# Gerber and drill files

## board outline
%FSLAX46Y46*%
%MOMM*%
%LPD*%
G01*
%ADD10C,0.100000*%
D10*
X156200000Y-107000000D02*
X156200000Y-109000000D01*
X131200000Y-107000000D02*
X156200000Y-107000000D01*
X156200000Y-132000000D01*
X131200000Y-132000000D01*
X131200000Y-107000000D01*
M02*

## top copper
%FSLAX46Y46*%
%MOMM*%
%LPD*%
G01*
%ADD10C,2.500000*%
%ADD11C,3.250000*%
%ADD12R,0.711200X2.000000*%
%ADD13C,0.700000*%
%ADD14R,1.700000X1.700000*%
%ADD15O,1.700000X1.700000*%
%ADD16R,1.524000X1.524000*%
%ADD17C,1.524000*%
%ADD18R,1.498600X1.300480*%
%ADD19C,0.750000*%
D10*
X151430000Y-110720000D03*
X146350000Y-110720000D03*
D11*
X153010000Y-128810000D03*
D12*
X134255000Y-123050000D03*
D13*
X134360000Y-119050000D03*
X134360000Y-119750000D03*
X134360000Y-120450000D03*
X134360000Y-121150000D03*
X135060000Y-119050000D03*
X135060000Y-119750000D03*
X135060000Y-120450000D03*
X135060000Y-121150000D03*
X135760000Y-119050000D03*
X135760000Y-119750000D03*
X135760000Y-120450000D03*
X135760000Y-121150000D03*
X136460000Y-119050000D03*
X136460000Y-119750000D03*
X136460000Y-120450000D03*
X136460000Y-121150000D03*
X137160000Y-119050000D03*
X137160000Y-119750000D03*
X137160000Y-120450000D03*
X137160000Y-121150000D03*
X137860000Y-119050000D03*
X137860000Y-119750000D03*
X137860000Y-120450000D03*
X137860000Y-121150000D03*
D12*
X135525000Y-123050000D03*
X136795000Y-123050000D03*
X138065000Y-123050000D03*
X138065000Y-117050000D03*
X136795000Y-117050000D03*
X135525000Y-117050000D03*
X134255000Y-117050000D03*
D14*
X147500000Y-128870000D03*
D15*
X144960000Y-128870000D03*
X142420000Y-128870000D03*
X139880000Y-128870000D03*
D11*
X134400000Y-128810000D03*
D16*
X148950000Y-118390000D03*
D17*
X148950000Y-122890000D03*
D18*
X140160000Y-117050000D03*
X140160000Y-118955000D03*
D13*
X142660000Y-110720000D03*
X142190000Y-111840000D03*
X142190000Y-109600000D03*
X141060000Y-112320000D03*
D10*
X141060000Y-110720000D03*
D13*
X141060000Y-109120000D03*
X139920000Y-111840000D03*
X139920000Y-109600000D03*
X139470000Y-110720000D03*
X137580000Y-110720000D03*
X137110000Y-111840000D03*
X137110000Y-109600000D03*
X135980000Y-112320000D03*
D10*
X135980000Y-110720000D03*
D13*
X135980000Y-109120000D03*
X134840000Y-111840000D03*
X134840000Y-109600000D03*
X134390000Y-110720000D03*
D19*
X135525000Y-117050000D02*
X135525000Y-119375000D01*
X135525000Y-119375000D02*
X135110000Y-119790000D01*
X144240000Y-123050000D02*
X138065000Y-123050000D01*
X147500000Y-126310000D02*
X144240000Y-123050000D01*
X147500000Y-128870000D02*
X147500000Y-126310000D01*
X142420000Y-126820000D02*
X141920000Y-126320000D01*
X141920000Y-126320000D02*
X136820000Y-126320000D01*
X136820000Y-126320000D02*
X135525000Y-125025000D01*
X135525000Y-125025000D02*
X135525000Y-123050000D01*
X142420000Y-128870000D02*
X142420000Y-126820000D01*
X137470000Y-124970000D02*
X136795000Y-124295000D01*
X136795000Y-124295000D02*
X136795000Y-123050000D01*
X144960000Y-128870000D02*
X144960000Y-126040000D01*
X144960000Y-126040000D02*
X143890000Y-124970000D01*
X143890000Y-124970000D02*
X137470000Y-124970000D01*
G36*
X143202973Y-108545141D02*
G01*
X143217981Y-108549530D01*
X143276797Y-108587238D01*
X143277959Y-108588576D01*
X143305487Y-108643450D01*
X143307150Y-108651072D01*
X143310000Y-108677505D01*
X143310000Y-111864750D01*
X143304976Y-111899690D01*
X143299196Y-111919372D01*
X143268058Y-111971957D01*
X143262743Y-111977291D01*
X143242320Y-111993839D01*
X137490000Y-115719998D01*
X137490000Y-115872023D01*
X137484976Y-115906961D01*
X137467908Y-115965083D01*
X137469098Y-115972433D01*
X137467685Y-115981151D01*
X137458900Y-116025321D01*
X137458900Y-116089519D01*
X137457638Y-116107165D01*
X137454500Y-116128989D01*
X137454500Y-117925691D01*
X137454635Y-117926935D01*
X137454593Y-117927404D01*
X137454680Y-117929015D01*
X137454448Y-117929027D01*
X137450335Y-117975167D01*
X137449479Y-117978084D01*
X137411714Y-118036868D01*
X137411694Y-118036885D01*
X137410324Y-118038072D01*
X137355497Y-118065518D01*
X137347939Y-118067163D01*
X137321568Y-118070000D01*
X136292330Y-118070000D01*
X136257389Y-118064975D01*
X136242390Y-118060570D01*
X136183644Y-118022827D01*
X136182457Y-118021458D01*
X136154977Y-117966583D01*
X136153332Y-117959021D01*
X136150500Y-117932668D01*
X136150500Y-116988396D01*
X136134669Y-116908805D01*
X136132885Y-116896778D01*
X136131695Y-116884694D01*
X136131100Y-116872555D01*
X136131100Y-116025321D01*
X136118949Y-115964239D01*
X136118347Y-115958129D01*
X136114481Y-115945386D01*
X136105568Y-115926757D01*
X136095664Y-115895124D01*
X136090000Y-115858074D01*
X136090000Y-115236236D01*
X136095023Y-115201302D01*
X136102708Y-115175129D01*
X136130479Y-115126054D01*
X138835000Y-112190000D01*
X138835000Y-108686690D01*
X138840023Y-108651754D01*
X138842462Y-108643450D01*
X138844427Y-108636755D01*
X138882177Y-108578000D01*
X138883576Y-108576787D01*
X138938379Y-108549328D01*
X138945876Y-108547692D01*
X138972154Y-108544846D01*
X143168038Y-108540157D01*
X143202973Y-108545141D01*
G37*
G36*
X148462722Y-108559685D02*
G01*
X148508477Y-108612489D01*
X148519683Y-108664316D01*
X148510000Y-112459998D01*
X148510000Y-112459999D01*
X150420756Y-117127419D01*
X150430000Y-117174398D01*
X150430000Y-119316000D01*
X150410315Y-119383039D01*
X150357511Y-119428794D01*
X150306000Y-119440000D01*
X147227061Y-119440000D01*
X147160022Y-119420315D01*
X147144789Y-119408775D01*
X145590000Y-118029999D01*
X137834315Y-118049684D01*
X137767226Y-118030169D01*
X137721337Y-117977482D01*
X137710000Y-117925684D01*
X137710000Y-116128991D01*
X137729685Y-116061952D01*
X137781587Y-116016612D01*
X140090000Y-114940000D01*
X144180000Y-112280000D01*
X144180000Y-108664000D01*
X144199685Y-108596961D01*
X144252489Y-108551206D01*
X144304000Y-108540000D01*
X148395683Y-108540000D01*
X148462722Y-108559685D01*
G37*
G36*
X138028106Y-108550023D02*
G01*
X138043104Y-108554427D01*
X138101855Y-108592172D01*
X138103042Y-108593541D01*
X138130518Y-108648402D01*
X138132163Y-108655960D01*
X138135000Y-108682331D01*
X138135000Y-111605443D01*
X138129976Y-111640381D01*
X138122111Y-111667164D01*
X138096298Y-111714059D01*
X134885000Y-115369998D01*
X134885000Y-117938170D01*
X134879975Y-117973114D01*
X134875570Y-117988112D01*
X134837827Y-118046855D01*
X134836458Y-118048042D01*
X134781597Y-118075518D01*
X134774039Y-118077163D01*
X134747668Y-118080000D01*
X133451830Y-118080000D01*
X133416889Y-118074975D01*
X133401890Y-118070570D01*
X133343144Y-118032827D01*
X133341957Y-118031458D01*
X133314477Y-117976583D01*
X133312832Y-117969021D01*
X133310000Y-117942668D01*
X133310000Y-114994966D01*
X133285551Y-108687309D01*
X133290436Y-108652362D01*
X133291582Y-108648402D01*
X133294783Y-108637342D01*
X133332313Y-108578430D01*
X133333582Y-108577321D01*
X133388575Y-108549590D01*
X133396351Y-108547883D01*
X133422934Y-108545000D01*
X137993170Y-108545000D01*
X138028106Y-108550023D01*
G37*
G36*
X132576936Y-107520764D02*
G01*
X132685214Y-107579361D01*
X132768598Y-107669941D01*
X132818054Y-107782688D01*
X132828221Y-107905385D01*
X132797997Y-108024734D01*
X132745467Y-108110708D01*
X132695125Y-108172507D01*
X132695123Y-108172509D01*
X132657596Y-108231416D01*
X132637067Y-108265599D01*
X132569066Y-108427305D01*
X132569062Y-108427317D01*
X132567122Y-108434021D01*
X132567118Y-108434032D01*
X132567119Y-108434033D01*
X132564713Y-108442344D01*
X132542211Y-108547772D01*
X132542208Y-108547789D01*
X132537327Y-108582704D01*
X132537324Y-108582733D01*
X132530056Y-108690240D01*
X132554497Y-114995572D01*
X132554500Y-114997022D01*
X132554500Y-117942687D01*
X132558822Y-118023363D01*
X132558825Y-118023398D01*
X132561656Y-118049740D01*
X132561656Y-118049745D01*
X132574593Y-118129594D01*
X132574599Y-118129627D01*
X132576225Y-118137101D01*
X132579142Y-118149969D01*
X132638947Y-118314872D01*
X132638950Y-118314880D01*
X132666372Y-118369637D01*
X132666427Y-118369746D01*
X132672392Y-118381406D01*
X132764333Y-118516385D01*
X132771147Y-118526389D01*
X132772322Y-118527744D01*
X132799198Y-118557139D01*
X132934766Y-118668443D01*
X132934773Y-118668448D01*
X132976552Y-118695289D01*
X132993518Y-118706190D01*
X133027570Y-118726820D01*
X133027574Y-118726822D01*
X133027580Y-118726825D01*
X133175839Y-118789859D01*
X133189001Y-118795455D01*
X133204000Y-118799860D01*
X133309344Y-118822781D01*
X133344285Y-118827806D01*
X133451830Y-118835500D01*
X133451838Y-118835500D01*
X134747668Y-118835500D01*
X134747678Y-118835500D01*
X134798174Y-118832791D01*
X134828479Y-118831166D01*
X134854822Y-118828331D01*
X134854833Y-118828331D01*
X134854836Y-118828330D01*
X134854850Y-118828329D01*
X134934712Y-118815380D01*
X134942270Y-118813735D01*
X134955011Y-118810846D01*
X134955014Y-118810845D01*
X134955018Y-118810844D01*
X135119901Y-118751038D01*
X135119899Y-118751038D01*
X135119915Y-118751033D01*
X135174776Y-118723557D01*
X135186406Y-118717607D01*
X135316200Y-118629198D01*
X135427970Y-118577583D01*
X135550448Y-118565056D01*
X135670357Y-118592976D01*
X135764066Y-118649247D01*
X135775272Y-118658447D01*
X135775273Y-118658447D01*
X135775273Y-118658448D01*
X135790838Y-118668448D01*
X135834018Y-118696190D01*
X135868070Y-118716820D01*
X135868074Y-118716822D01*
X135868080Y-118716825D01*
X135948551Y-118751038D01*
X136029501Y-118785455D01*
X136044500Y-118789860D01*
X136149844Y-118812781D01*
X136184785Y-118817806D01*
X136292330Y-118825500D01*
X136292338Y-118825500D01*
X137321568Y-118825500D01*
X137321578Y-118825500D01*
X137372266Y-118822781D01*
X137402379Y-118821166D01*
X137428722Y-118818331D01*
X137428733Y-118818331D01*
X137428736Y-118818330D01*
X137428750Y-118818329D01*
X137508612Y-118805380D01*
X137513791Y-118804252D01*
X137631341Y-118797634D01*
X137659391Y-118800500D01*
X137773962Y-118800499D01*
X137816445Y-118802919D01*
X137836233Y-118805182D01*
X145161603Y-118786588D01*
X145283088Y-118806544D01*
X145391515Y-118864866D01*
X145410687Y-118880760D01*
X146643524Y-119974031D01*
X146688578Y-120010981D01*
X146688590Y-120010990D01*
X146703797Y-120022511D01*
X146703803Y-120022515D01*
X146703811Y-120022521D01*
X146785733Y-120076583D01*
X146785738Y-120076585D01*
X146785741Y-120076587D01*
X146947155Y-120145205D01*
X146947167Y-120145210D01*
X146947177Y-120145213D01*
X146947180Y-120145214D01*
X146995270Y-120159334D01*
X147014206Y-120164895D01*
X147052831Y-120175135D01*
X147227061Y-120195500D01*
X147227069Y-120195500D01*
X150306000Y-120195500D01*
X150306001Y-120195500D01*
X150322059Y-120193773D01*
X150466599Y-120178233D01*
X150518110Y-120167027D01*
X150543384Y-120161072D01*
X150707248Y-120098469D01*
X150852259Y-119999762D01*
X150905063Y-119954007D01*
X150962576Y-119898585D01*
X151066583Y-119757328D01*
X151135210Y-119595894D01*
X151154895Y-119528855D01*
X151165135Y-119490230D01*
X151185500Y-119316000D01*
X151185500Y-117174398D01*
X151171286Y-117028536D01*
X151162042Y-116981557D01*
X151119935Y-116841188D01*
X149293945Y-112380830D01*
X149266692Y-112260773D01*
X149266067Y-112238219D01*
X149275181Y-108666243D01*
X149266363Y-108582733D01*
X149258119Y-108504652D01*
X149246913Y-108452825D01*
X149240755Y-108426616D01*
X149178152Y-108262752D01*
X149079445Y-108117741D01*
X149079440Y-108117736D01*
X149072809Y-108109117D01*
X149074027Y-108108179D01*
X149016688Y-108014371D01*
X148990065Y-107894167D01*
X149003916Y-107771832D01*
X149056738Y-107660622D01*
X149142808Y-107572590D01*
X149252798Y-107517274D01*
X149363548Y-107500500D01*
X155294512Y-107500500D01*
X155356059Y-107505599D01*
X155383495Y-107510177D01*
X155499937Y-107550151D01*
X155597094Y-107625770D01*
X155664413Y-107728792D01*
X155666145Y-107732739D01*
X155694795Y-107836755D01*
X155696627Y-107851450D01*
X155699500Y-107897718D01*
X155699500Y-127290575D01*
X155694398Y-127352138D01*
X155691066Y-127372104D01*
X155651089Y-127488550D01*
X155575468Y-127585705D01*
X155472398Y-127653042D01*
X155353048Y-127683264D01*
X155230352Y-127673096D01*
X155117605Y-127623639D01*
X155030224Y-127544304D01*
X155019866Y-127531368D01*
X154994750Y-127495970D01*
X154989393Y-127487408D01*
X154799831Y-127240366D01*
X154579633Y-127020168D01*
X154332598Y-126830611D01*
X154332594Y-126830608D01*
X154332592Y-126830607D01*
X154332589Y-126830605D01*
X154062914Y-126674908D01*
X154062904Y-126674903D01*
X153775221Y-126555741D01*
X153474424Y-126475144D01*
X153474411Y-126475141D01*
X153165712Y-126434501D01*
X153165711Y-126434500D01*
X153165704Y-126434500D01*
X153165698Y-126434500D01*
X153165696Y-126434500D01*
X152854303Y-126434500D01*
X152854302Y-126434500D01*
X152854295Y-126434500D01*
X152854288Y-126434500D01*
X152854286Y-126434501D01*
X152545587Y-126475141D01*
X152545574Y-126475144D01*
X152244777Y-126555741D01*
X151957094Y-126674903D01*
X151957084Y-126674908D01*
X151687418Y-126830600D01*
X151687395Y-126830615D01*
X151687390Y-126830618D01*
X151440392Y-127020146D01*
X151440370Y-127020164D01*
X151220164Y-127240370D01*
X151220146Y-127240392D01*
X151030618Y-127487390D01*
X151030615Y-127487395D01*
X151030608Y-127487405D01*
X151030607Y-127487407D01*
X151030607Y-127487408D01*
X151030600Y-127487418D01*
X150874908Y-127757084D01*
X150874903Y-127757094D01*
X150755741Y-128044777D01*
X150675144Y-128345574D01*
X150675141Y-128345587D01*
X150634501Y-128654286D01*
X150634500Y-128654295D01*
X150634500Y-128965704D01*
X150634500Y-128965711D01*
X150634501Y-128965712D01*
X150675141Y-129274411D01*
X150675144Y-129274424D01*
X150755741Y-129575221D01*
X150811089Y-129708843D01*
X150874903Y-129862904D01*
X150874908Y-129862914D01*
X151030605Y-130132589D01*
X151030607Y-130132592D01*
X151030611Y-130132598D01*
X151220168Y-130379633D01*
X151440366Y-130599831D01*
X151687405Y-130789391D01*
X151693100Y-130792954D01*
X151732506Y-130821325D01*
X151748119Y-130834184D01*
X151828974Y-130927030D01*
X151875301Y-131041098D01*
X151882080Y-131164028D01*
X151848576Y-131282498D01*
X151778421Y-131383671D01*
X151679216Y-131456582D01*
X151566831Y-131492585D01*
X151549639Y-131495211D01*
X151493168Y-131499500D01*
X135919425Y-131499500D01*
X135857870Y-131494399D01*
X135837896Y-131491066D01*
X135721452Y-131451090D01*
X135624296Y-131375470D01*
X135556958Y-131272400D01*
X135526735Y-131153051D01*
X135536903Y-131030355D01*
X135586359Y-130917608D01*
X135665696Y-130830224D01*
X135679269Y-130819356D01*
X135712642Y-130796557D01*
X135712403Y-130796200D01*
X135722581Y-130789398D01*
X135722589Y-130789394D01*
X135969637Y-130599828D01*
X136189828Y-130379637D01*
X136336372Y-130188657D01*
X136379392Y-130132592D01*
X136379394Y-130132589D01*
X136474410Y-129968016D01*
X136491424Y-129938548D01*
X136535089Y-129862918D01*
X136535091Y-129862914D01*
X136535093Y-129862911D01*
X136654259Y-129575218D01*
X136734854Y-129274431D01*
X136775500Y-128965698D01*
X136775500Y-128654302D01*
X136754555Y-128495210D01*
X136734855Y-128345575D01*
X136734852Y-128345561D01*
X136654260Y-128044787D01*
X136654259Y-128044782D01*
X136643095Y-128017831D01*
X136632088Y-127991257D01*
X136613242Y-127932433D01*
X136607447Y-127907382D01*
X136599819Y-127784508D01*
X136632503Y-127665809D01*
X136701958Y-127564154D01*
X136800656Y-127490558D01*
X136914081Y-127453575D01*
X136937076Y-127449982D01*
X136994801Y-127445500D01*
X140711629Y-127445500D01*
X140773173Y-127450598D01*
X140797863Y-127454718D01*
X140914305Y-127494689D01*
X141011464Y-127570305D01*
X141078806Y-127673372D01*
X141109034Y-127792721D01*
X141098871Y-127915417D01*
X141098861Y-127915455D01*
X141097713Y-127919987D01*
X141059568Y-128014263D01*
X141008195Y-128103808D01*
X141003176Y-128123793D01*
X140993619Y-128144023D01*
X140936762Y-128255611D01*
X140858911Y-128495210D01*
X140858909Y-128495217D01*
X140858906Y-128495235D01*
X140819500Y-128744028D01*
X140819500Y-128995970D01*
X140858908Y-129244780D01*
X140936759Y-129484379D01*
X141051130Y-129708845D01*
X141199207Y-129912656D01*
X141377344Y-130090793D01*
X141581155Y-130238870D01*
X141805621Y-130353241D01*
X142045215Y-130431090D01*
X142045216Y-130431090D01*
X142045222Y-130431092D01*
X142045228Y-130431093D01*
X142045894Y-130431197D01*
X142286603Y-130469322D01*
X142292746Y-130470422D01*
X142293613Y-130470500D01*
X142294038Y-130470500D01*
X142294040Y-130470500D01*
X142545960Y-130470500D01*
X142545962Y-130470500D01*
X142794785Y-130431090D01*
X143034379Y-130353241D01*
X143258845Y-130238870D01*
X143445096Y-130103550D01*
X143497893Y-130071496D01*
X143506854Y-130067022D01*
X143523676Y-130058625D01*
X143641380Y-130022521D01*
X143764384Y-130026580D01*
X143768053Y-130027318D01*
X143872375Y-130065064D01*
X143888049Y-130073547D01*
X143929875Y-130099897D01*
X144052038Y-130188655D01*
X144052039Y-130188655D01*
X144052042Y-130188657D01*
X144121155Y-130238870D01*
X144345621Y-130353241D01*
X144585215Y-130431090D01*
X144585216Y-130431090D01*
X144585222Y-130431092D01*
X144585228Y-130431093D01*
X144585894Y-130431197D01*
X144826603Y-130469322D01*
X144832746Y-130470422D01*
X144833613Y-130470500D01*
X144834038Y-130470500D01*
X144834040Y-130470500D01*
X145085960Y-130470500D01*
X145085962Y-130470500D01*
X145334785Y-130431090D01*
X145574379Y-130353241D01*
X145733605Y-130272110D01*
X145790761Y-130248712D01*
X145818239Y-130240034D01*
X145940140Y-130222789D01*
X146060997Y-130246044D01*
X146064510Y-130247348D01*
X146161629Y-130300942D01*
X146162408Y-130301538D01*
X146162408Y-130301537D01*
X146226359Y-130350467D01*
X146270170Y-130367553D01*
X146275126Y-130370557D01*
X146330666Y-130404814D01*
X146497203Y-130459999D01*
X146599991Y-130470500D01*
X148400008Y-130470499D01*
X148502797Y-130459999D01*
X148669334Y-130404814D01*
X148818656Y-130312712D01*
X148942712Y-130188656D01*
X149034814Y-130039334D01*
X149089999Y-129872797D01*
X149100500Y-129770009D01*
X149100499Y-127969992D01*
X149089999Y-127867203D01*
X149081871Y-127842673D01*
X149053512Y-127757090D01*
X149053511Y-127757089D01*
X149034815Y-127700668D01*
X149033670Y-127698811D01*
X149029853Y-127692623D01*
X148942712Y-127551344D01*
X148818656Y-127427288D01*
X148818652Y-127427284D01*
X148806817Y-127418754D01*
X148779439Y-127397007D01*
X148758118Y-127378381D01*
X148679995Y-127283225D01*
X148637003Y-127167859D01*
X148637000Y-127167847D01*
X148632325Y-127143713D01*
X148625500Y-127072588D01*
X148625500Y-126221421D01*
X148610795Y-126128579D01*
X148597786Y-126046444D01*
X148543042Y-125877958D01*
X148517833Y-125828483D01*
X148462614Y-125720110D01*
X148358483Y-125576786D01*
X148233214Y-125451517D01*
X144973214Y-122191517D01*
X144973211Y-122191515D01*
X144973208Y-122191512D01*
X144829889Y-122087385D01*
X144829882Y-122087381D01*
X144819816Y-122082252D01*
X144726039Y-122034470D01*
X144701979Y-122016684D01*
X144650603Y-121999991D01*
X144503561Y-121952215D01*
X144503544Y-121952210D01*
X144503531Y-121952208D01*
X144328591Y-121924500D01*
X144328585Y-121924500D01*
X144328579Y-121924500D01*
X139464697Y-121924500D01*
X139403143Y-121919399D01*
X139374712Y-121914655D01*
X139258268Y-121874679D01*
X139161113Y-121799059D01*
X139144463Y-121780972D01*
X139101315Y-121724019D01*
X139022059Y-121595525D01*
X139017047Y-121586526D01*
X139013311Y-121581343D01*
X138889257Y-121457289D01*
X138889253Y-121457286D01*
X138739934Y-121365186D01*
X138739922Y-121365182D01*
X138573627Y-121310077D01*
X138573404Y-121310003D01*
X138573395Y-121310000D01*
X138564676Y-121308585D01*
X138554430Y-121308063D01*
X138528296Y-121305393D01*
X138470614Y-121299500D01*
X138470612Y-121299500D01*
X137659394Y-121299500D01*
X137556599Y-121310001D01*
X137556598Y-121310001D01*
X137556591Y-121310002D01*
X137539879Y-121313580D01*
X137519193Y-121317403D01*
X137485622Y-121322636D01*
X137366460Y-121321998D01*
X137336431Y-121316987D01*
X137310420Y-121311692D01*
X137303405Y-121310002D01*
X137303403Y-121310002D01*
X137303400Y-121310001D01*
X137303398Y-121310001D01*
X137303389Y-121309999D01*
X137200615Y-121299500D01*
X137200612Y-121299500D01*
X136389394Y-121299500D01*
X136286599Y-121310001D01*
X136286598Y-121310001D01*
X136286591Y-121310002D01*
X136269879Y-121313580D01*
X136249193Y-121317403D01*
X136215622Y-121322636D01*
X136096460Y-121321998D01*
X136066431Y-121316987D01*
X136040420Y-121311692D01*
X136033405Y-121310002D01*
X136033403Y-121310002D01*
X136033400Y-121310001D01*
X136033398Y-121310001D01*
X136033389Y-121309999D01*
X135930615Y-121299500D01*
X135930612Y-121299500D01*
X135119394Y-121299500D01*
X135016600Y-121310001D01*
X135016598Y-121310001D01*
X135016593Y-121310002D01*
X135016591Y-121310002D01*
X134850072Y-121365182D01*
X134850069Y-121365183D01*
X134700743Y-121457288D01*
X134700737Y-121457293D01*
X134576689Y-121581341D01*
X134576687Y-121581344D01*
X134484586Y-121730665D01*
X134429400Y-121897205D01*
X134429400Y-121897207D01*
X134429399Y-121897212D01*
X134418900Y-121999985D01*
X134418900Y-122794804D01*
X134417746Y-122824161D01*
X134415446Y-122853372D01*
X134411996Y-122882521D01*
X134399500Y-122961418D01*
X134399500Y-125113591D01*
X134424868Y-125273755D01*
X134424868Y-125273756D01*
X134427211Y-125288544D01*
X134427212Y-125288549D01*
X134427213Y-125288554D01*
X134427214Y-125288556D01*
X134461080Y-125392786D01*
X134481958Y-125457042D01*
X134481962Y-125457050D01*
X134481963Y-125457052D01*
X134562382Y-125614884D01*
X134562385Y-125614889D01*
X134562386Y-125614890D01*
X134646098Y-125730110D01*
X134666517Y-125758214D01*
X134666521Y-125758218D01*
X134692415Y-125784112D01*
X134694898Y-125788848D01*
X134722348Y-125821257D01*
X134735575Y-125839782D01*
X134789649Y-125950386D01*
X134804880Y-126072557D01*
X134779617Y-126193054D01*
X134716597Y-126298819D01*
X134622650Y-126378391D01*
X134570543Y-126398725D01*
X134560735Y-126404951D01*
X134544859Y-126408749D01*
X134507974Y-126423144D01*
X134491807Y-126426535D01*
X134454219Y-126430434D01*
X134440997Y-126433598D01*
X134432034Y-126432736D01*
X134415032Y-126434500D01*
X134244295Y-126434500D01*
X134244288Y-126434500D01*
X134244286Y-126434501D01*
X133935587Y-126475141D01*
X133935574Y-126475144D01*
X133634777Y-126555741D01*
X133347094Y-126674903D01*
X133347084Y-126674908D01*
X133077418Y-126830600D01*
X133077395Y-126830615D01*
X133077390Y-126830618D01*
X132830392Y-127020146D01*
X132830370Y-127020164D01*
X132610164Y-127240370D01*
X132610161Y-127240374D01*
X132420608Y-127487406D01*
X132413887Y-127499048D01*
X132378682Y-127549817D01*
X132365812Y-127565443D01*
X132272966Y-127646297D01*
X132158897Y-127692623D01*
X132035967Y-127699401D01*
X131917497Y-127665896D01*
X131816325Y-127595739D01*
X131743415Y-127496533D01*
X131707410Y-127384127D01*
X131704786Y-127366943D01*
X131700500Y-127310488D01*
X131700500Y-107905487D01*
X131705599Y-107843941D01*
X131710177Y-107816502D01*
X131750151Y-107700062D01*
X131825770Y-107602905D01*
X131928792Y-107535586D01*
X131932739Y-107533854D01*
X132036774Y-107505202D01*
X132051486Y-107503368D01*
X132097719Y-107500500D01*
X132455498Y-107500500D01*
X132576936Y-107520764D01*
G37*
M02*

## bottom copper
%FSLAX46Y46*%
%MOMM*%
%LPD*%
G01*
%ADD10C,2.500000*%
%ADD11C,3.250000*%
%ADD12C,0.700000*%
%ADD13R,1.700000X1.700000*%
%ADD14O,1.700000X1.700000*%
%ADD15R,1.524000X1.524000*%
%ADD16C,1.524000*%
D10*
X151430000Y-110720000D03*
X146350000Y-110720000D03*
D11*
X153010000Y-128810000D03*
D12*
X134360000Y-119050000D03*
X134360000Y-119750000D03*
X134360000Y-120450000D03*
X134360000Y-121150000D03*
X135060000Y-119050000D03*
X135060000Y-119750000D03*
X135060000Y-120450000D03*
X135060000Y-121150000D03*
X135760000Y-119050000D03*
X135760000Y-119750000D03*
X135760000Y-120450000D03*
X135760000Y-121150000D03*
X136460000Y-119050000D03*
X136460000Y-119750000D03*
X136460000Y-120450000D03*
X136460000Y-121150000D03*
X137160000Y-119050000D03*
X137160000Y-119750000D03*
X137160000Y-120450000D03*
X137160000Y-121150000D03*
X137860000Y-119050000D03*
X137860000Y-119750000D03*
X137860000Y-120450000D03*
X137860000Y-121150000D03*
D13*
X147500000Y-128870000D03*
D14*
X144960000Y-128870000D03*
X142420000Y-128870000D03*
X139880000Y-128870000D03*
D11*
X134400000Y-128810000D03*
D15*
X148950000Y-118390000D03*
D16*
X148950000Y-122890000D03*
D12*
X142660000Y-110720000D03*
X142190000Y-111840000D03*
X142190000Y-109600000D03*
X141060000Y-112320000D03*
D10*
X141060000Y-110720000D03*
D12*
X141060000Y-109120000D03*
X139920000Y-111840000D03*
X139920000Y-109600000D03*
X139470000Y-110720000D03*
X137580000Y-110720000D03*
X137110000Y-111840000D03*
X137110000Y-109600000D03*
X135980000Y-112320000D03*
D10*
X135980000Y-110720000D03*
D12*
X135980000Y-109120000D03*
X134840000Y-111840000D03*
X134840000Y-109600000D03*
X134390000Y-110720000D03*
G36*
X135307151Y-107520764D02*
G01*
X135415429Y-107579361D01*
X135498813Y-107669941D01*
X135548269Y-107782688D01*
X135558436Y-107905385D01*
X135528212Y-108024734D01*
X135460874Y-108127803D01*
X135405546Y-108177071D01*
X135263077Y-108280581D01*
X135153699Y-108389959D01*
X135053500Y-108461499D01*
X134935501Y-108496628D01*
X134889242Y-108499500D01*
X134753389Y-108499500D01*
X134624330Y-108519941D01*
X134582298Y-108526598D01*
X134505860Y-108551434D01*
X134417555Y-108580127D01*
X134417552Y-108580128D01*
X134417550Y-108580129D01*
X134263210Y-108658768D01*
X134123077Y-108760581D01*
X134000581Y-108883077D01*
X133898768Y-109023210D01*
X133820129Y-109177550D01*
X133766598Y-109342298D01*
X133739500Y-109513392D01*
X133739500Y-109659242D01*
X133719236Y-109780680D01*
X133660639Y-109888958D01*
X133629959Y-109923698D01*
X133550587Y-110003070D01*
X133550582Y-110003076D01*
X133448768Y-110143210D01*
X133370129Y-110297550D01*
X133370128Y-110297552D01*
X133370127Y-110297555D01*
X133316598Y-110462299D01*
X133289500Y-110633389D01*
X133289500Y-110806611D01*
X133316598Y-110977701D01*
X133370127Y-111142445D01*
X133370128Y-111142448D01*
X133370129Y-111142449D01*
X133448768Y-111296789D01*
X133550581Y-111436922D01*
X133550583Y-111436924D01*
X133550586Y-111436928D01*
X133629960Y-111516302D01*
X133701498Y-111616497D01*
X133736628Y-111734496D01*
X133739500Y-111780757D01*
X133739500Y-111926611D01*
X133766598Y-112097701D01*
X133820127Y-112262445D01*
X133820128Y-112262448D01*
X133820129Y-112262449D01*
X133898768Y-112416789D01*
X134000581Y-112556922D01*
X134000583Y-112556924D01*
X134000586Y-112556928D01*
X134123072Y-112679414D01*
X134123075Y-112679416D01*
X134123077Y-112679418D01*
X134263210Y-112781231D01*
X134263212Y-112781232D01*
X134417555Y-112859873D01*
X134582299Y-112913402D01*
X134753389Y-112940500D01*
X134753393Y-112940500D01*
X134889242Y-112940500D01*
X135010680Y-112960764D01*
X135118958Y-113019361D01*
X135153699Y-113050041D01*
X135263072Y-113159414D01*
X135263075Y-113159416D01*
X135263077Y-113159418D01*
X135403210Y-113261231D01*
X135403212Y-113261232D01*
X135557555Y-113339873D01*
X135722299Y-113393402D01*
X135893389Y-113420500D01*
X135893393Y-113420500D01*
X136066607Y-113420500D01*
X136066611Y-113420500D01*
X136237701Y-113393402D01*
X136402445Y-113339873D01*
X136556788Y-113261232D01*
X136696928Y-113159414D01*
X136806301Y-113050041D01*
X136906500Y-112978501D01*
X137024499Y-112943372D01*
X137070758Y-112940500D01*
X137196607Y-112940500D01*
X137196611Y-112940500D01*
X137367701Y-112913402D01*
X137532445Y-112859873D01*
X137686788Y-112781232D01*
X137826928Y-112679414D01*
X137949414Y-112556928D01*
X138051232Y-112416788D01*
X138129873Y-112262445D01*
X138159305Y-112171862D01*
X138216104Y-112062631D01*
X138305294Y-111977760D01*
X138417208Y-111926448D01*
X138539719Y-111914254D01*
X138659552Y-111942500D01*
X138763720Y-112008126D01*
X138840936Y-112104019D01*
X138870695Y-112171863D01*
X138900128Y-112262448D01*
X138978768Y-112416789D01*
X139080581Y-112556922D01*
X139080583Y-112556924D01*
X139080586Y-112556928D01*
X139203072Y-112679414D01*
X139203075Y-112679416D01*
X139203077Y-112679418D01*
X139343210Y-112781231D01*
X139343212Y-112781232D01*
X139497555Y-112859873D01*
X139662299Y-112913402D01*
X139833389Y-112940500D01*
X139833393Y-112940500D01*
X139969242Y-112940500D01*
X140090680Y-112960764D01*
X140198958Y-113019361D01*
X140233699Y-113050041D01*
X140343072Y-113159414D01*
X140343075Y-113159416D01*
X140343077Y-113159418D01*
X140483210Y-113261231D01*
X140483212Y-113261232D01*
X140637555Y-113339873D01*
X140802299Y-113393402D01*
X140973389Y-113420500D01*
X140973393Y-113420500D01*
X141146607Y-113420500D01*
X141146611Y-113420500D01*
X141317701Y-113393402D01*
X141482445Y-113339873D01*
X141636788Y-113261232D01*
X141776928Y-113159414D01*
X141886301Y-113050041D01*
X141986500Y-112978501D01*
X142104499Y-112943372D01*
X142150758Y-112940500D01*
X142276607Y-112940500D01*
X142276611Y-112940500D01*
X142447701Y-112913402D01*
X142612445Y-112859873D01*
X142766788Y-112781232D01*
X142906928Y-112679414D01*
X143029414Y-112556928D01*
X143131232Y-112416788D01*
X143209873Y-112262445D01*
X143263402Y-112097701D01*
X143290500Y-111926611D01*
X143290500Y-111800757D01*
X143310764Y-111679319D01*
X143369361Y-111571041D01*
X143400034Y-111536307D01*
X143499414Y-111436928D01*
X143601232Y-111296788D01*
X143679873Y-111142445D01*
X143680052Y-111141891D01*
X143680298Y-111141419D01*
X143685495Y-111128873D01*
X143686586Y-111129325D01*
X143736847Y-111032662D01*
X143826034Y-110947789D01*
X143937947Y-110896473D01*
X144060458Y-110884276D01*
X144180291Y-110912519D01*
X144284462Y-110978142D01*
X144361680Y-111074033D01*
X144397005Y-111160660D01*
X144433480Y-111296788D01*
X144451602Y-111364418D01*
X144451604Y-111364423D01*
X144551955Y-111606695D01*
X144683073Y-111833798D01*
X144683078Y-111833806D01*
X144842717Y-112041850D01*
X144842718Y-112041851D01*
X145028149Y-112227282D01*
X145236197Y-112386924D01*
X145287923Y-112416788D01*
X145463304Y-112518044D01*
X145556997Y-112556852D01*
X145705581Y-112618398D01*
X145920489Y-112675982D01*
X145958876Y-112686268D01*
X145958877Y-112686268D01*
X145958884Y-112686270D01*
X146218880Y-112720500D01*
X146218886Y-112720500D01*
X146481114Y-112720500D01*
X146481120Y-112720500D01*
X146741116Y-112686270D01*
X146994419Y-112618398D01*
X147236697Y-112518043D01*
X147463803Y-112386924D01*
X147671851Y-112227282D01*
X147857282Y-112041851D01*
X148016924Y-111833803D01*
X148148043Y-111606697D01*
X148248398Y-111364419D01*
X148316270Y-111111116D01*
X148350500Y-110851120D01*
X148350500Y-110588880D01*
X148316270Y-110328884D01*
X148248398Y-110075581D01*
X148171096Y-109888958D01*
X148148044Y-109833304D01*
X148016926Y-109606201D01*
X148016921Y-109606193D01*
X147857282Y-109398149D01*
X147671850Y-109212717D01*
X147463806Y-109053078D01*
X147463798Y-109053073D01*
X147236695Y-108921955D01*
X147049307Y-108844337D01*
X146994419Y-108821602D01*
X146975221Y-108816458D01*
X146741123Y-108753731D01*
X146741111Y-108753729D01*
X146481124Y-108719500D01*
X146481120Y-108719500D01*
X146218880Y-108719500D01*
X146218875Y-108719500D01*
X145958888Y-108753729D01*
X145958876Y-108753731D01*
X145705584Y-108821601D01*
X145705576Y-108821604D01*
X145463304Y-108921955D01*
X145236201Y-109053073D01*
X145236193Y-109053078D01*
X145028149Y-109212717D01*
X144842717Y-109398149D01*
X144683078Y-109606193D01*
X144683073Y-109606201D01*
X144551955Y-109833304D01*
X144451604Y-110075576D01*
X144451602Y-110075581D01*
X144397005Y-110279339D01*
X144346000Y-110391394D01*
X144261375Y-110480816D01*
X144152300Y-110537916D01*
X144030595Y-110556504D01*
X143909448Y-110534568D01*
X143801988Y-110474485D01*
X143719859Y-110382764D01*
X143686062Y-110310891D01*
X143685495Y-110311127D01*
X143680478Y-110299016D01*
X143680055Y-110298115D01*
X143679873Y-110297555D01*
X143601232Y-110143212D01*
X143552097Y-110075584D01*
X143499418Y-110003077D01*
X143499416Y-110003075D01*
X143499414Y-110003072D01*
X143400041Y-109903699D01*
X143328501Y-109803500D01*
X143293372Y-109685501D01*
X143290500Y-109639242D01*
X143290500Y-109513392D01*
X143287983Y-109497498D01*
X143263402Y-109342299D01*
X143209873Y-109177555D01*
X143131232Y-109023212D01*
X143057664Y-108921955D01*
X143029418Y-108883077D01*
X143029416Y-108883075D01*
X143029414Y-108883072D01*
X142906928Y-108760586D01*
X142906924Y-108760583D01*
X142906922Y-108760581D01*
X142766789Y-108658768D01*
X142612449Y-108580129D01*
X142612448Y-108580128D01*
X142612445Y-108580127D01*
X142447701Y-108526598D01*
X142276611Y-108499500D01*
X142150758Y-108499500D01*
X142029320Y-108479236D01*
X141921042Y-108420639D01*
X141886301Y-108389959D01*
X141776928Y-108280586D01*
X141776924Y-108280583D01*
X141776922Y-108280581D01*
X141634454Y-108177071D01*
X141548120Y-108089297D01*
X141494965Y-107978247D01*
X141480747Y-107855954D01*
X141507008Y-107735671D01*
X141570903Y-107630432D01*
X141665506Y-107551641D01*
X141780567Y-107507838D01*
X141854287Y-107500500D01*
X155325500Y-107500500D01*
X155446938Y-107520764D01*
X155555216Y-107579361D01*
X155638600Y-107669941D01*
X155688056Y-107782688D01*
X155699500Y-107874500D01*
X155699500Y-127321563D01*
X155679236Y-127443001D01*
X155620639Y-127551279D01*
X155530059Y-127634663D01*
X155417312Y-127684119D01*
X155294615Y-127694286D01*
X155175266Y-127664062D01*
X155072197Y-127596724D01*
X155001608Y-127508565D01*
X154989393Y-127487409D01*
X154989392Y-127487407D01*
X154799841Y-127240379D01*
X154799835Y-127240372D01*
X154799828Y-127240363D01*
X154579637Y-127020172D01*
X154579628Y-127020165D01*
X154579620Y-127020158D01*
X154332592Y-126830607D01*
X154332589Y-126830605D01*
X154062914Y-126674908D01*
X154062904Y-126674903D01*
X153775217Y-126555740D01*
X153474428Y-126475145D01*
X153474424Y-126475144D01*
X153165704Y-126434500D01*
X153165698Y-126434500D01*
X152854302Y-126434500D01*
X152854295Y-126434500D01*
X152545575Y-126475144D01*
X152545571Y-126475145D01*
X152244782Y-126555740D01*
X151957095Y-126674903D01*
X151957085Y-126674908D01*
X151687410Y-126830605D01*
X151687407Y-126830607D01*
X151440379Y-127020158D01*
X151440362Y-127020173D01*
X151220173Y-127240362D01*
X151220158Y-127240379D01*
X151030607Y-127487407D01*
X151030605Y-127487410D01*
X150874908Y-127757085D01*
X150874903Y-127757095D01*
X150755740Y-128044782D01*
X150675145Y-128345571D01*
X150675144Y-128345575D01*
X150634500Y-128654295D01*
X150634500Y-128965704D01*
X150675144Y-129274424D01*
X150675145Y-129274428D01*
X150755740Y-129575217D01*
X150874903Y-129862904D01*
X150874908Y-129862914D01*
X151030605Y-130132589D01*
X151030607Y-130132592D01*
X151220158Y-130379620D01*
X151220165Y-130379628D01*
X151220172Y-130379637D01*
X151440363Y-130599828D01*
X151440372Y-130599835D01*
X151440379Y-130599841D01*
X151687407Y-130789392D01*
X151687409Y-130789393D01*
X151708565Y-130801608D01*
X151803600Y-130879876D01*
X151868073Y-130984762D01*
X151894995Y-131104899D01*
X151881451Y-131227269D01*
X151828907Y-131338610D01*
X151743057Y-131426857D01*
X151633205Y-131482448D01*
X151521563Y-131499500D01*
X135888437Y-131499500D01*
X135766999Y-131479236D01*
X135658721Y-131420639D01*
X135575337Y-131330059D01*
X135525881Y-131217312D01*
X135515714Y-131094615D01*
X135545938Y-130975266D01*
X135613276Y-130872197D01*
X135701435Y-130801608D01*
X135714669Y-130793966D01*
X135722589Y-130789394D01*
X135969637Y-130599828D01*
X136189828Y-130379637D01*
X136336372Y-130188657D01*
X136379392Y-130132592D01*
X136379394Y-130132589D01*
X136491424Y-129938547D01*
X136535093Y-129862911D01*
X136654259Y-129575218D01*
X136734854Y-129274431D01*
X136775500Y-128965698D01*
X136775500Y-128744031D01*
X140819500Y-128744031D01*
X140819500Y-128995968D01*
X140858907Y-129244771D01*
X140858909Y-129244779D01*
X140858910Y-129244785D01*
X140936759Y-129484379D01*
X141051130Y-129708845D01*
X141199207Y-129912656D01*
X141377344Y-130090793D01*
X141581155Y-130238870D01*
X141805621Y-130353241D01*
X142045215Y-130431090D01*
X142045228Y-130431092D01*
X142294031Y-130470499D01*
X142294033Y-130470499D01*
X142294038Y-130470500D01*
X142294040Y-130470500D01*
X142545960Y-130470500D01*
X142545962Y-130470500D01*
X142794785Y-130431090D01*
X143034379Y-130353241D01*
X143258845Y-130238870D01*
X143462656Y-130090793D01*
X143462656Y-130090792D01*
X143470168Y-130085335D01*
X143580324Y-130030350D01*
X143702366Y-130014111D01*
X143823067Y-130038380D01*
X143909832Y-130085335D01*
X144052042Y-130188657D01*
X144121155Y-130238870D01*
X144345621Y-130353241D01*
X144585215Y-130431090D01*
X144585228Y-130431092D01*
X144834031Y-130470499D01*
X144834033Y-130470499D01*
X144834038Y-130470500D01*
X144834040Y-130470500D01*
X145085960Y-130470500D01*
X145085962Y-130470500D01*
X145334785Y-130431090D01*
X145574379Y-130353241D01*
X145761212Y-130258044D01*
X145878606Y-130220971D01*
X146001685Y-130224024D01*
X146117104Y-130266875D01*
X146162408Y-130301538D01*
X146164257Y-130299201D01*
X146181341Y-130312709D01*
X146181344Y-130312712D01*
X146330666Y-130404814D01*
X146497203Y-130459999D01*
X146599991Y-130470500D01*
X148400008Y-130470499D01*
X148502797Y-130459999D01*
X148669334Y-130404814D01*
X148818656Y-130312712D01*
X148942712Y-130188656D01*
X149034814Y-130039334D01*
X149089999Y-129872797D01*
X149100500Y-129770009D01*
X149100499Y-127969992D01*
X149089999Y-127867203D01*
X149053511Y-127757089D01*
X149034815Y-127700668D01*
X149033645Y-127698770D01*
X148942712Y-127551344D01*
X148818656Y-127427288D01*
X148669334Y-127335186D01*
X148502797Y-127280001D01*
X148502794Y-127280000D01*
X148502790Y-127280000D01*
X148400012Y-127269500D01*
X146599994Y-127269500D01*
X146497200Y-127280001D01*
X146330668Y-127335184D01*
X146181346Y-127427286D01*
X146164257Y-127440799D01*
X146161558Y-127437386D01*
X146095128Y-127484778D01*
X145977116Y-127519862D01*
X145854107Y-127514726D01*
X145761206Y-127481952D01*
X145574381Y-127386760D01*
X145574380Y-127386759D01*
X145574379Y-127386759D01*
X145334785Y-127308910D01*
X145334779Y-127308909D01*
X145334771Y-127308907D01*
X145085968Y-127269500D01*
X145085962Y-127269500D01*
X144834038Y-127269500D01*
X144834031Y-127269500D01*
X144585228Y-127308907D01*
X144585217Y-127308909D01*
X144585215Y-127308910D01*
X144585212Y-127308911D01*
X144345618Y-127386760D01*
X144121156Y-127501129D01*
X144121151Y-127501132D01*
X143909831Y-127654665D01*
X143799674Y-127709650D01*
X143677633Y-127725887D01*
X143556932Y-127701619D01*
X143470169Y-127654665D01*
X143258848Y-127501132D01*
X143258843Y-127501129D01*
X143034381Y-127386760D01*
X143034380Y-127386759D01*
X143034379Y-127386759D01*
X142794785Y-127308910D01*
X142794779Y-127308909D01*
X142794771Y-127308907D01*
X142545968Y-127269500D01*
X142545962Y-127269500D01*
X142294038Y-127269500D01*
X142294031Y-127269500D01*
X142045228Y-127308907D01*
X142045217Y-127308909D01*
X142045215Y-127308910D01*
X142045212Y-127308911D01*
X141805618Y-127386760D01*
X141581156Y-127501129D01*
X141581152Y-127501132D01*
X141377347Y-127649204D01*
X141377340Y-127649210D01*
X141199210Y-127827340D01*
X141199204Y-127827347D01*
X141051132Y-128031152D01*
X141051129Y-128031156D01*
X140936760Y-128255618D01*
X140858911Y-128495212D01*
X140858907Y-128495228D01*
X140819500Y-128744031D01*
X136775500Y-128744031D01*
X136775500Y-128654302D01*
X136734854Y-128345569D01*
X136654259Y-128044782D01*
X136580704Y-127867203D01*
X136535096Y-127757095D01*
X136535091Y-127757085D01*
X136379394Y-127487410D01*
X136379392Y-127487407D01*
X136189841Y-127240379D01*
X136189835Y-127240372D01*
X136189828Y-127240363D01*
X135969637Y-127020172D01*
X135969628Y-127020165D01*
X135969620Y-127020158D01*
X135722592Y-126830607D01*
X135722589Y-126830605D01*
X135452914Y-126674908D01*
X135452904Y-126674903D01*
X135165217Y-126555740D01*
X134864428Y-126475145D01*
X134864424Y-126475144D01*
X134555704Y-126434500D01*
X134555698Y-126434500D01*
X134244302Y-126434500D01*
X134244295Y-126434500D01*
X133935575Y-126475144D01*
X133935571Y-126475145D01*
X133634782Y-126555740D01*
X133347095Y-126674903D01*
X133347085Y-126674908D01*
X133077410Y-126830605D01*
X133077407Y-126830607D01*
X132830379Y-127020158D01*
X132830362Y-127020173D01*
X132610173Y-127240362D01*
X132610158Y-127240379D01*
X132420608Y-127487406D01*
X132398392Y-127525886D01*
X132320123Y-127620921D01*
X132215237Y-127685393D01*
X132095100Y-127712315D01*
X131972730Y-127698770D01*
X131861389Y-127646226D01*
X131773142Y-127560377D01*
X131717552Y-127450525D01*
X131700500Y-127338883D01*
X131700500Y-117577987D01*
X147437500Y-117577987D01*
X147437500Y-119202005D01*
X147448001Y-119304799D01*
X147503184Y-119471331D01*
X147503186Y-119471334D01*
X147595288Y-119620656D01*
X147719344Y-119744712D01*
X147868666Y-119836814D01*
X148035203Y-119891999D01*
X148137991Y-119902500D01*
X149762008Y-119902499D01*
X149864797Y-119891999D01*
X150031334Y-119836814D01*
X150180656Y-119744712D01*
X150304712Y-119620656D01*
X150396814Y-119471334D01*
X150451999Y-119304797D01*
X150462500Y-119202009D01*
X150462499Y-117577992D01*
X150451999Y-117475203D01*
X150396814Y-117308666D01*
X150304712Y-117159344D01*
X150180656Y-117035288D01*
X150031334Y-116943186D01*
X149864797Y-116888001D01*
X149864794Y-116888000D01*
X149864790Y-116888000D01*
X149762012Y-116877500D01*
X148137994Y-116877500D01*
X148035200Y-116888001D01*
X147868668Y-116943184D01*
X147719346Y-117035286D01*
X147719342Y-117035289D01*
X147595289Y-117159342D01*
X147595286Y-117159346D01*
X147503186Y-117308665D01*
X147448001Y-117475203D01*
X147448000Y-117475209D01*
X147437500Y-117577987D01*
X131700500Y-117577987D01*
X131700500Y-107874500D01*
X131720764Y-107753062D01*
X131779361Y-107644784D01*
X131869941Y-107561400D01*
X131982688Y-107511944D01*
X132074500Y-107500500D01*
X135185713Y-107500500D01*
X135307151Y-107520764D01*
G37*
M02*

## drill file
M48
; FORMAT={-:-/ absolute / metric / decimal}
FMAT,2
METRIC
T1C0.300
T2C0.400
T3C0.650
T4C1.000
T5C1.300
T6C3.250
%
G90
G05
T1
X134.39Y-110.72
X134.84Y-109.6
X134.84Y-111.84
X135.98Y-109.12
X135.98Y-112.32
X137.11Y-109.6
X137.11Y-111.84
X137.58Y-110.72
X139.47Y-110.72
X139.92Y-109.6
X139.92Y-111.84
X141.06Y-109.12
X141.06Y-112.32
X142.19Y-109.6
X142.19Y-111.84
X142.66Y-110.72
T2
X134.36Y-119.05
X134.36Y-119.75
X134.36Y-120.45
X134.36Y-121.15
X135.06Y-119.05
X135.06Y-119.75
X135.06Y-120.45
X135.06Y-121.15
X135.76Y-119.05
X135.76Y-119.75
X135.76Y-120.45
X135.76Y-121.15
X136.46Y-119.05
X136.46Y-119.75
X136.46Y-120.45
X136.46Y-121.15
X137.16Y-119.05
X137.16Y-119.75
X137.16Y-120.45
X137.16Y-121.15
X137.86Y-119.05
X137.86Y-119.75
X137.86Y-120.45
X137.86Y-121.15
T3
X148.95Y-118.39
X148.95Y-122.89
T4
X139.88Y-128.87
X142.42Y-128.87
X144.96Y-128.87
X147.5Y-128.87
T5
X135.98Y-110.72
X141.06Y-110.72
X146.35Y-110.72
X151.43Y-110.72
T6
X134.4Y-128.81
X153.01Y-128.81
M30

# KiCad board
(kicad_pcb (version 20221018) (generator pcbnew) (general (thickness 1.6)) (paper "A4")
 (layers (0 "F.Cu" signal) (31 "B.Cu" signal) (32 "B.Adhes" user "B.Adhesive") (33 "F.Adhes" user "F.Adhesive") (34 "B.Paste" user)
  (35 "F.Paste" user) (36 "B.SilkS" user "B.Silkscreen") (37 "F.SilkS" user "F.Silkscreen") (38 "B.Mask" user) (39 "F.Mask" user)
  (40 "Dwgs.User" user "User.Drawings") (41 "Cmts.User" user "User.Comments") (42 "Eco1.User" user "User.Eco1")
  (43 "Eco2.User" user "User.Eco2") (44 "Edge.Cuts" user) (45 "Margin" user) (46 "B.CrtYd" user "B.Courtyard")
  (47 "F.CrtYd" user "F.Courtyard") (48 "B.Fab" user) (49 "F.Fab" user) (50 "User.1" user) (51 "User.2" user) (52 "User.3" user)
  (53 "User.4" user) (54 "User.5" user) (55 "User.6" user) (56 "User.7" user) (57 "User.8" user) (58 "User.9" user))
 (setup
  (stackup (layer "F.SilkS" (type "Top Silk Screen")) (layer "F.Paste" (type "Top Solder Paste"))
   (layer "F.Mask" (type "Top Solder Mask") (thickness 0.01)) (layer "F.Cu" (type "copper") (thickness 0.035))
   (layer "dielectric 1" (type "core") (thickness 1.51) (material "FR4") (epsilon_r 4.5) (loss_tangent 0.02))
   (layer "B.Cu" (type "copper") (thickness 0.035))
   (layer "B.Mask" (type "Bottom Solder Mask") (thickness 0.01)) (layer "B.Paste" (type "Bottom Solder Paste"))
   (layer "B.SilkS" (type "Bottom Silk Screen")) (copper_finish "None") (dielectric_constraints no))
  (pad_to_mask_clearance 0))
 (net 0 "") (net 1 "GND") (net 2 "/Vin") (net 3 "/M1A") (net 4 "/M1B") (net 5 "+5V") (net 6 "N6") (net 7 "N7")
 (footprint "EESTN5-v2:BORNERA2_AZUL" (layer "F.Cu") (at 148.89 110.72 180)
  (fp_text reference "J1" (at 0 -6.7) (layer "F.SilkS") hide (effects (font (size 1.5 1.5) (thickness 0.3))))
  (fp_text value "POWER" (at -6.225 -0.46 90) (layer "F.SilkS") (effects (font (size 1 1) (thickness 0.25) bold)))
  (pad "1" thru_hole circle (at -2.54 0 180) (size 2.5 2.5) (drill 1.3) (layers "*.Cu" "*.Mask" "F.SilkS") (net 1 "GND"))
  (pad "2" thru_hole circle (at 2.54 0 180) (size 2.5 2.5) (drill 1.3) (layers "*.Cu" "*.Mask" "F.SilkS") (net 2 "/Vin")))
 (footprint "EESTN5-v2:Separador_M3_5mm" (layer "F.Cu") (at 153.01 128.81)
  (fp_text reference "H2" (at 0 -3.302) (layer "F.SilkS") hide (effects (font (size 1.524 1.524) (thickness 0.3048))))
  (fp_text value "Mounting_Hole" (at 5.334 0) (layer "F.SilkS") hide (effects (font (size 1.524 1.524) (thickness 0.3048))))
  (pad "1" thru_hole circle (at 0 0) (size 3.25 3.25) (drill 3.25) (layers "*.Cu" "F.SilkS")))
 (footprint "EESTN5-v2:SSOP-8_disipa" (layer "F.Cu") (at 136.16 120.05)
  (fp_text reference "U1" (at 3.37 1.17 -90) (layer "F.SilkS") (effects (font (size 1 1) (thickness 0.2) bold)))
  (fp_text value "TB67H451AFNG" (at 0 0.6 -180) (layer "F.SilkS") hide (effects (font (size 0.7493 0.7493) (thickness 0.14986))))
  (pad "1" smd rect (at -1.905 3) (size 0.7112 2) (layers "F.Cu" "F.Paste" "F.Mask") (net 1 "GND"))
  (pad "1" thru_hole circle (at -1.8 -1 90) (size 0.7 0.7) (drill 0.4) (layers "*.Cu" "*.Mask") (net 1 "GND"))
  (pad "1" thru_hole circle (at -1.8 -0.3 90) (size 0.7 0.7) (drill 0.4) (layers "*.Cu" "*.Mask") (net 1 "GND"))
  (pad "1" thru_hole circle (at -1.8 0.4 90) (size 0.7 0.7) (drill 0.4) (layers "*.Cu" "*.Mask") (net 1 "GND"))
  (pad "1" thru_hole circle (at -1.8 1.1 90) (size 0.7 0.7) (drill 0.4) (layers "*.Cu" "*.Mask") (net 1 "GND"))
  (pad "1" thru_hole circle (at -1.1 -1 90) (size 0.7 0.7) (drill 0.4) (layers "*.Cu" "*.Mask") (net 1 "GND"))
  (pad "1" thru_hole circle (at -1.1 -0.3 90) (size 0.7 0.7) (drill 0.4) (layers "*.Cu" "*.Mask") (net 1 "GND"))
  (pad "1" thru_hole circle (at -1.1 0.4 90) (size 0.7 0.7) (drill 0.4) (layers "*.Cu" "*.Mask") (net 1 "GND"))
  (pad "1" thru_hole circle (at -1.1 1.1 90) (size 0.7 0.7) (drill 0.4) (layers "*.Cu" "*.Mask") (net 1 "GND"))
  (pad "1" thru_hole circle (at -0.4 -1) (size 0.7 0.7) (drill 0.4) (layers "*.Cu" "*.Mask") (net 1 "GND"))
  (pad "1" thru_hole circle (at -0.4 -0.3) (size 0.7 0.7) (drill 0.4) (layers "*.Cu" "*.Mask") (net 1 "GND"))
  (pad "1" thru_hole circle (at -0.4 0.4) (size 0.7 0.7) (drill 0.4) (layers "*.Cu" "*.Mask") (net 1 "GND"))
  (pad "1" thru_hole circle (at -0.4 1.1) (size 0.7 0.7) (drill 0.4) (layers "*.Cu" "*.Mask") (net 1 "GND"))
  (pad "1" thru_hole circle (at 0.3 -1) (size 0.7 0.7) (drill 0.4) (layers "*.Cu" "*.Mask") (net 1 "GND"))
  (pad "1" thru_hole circle (at 0.3 -0.3) (size 0.7 0.7) (drill 0.4) (layers "*.Cu" "*.Mask") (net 1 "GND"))
  (pad "1" thru_hole circle (at 0.3 0.4) (size 0.7 0.7) (drill 0.4) (layers "*.Cu" "*.Mask") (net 1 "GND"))
  (pad "1" thru_hole circle (at 0.3 1.1) (size 0.7 0.7) (drill 0.4) (layers "*.Cu" "*.Mask") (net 1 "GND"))
  (pad "1" thru_hole circle (at 1 -1) (size 0.7 0.7) (drill 0.4) (layers "*.Cu" "*.Mask") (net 1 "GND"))
  (pad "1" thru_hole circle (at 1 -0.3) (size 0.7 0.7) (drill 0.4) (layers "*.Cu" "*.Mask") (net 1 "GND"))
  (pad "1" thru_hole circle (at 1 0.4) (size 0.7 0.7) (drill 0.4) (layers "*.Cu" "*.Mask") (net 1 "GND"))
  (pad "1" thru_hole circle (at 1 1.1) (size 0.7 0.7) (drill 0.4) (layers "*.Cu" "*.Mask") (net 1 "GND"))
  (pad "1" thru_hole circle (at 1.7 -1) (size 0.7 0.7) (drill 0.4) (layers "*.Cu" "*.Mask") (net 1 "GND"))
  (pad "1" thru_hole circle (at 1.7 -0.3) (size 0.7 0.7) (drill 0.4) (layers "*.Cu" "*.Mask") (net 1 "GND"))
  (pad "1" thru_hole circle (at 1.7 0.4) (size 0.7 0.7) (drill 0.4) (layers "*.Cu" "*.Mask") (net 1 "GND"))
  (pad "1" thru_hole circle (at 1.7 1.1) (size 0.7 0.7) (drill 0.4) (layers "*.Cu" "*.Mask") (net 1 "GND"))
  (pad "2" smd rect (at -0.635 3) (size 0.7112 2) (layers "F.Cu" "F.Paste" "F.Mask") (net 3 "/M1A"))
  (pad "3" smd rect (at 0.635 3) (size 0.7112 2) (layers "F.Cu" "F.Paste" "F.Mask") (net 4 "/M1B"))
  (pad "4" smd rect (at 1.905 3) (size 0.7112 2) (layers "F.Cu" "F.Paste" "F.Mask") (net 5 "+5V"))
  (pad "5" smd rect (at 1.905 -3 180) (size 0.7112 2) (layers "F.Cu" "F.Paste" "F.Mask") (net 2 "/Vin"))
  (pad "6" smd rect (at 0.635 -3 180) (size 0.7112 2) (layers "F.Cu" "F.Paste" "F.Mask") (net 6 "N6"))
  (pad "7" smd rect (at -0.635 -3 180) (size 0.7112 2) (layers "F.Cu" "F.Paste" "F.Mask") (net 1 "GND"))
  (pad "8" smd rect (at -1.905 -3 180) (size 0.7112 2) (layers "F.Cu" "F.Paste" "F.Mask") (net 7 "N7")))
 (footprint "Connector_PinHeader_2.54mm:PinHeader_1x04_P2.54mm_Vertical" (layer "F.Cu") (at 147.5 128.87 -90)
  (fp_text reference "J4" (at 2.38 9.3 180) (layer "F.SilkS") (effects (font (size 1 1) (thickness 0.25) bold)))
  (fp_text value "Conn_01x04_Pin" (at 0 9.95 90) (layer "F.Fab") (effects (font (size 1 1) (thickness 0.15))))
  (pad "1" thru_hole rect (at 0 0 270) (size 1.7 1.7) (drill 1) (layers "*.Cu" "*.Mask") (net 5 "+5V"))
  (pad "2" thru_hole oval (at 0 2.54 270) (size 1.7 1.7) (drill 1) (layers "*.Cu" "*.Mask") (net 4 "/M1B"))
  (pad "3" thru_hole oval (at 0 5.08 270) (size 1.7 1.7) (drill 1) (layers "*.Cu" "*.Mask") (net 3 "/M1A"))
  (pad "4" thru_hole oval (at 0 7.62 270) (size 1.7 1.7) (drill 1) (layers "*.Cu" "*.Mask") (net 1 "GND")))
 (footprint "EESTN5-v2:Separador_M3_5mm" (layer "F.Cu") (at 134.4 128.81)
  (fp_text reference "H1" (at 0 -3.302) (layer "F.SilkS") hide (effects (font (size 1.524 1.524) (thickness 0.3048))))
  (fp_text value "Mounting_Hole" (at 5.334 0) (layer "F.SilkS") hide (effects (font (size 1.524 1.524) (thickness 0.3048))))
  (pad "1" thru_hole circle (at 0 0) (size 3.25 3.25) (drill 3.25) (layers "*.Cu" "F.SilkS")))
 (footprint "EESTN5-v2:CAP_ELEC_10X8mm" (layer "F.Cu") (at 148.95 120.64 180)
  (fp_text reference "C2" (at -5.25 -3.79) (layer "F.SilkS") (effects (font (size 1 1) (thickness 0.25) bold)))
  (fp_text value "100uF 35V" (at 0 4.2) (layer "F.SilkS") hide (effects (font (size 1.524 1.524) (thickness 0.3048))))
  (pad "1" thru_hole rect (at 0 2.25 180) (size 1.524 1.524) (drill 0.65) (layers "*.Cu" "*.Mask" "F.SilkS") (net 2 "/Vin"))
  (pad "2" thru_hole circle (at 0 -2.25 180) (size 1.524 1.524) (drill 0.65) (layers "*.Cu" "*.Mask" "F.SilkS") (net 1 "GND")))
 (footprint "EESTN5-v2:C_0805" (layer "F.Cu") (at 140.16 118.0025 90)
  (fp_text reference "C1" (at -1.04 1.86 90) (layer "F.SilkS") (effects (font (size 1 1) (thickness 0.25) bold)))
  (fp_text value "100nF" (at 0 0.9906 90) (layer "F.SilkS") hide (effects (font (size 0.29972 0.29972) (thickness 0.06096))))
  (pad "1" smd rect (at 0.9525 0 90) (size 1.30048 1.4986) (layers "F.Cu" "F.Paste" "F.Mask") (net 2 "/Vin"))
  (pad "2" smd rect (at -0.9525 0 90) (size 1.30048 1.4986) (layers "F.Cu" "F.Paste" "F.Mask") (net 1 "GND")))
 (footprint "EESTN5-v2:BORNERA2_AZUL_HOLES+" (layer "F.Cu") (at 138.52 110.72 180)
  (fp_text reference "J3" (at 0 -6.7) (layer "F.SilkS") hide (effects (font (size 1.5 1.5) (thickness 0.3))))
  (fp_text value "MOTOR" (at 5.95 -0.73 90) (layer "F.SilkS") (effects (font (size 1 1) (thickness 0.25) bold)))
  (pad "1" thru_hole circle (at -4.14 0 180) (size 0.7 0.7) (drill 0.3) (layers "*.Cu" "*.Mask" "F.SilkS") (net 6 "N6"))
  (pad "1" thru_hole circle (at -3.67 -1.12 180) (size 0.7 0.7) (drill 0.3) (layers "*.Cu" "*.Mask" "F.SilkS") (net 6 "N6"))
  (pad "1" thru_hole circle (at -3.67 1.12 180) (size 0.7 0.7) (drill 0.3) (layers "*.Cu" "*.Mask" "F.SilkS") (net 6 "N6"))
  (pad "1" thru_hole circle (at -2.54 -1.6 180) (size 0.7 0.7) (drill 0.3) (layers "*.Cu" "*.Mask" "F.SilkS") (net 6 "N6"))
  (pad "1" thru_hole circle (at -2.54 0 180) (size 2.5 2.5) (drill 1.3) (layers "*.Cu" "*.Mask" "F.SilkS") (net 6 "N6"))
  (pad "1" thru_hole circle (at -2.54 1.6 180) (size 0.7 0.7) (drill 0.3) (layers "*.Cu" "*.Mask" "F.SilkS") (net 6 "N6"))
  (pad "1" thru_hole circle (at -1.4 -1.12 180) (size 0.7 0.7) (drill 0.3) (layers "*.Cu" "*.Mask" "F.SilkS") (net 6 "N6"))
  (pad "1" thru_hole circle (at -1.4 1.12 180) (size 0.7 0.7) (drill 0.3) (layers "*.Cu" "*.Mask" "F.SilkS") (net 6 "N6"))
  (pad "1" thru_hole circle (at -0.95 0 180) (size 0.7 0.7) (drill 0.3) (layers "*.Cu" "*.Mask" "F.SilkS") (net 6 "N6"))
  (pad "2" thru_hole circle (at 0.94 0 180) (size 0.7 0.7) (drill 0.3) (layers "*.Cu" "*.Mask" "F.SilkS") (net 7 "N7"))
  (pad "2" thru_hole circle (at 1.41 -1.12 180) (size 0.7 0.7) (drill 0.3) (layers "*.Cu" "*.Mask" "F.SilkS") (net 7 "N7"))
  (pad "2" thru_hole circle (at 1.41 1.12 180) (size 0.7 0.7) (drill 0.3) (layers "*.Cu" "*.Mask" "F.SilkS") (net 7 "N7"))
  (pad "2" thru_hole circle (at 2.54 -1.6 180) (size 0.7 0.7) (drill 0.3) (layers "*.Cu" "*.Mask" "F.SilkS") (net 7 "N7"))
  (pad "2" thru_hole circle (at 2.54 0 180) (size 2.5 2.5) (drill 1.3) (layers "*.Cu" "*.Mask" "F.SilkS") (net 7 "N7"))
  (pad "2" thru_hole circle (at 2.54 1.6 180) (size 0.7 0.7) (drill 0.3) (layers "*.Cu" "*.Mask" "F.SilkS") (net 7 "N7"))
  (pad "2" thru_hole circle (at 3.68 -1.12 180) (size 0.7 0.7) (drill 0.3) (layers "*.Cu" "*.Mask" "F.SilkS") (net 7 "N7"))
  (pad "2" thru_hole circle (at 3.68 1.12 180) (size 0.7 0.7) (drill 0.3) (layers "*.Cu" "*.Mask" "F.SilkS") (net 7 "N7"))
  (pad "2" thru_hole circle (at 4.13 0 180) (size 0.7 0.7) (drill 0.3) (layers "*.Cu" "*.Mask" "F.SilkS") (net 7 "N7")))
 (gr_line (start 156.2 107) (end 156.2 109) (stroke (width 0.1) (type default)) (layer "Edge.Cuts"))
 (gr_rect (start 131.2 107) (end 156.2 132) (stroke (width 0.1) (type default)) (fill none) (layer "Edge.Cuts"))
 (segment (start 135.525 117.05) (end 135.525 119.375) (width 0.75) (layer "F.Cu") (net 1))
 (segment (start 135.525 119.375) (end 135.11 119.79) (width 0.75) (layer "F.Cu") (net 1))
 (segment (start 144.24 123.05) (end 138.065 123.05) (width 0.75) (layer "F.Cu") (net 5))
 (segment (start 147.5 126.31) (end 144.24 123.05) (width 0.75) (layer "F.Cu") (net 5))
 (segment (start 147.5 128.87) (end 147.5 126.31) (width 0.75) (layer "F.Cu") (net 5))
 (segment (start 142.42 126.82) (end 141.92 126.32) (width 0.75) (layer "F.Cu") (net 3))
 (segment (start 141.92 126.32) (end 136.82 126.32) (width 0.75) (layer "F.Cu") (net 3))
 (segment (start 136.82 126.32) (end 135.525 125.025) (width 0.75) (layer "F.Cu") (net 3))
 (segment (start 135.525 125.025) (end 135.525 123.05) (width 0.75) (layer "F.Cu") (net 3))
 (segment (start 142.42 128.87) (end 142.42 126.82) (width 0.75) (layer "F.Cu") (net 3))
 (segment (start 137.47 124.97) (end 136.795 124.295) (width 0.75) (layer "F.Cu") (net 4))
 (segment (start 136.795 124.295) (end 136.795 123.05) (width 0.75) (layer "F.Cu") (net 4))
 (segment (start 144.96 128.87) (end 144.96 126.04) (width 0.75) (layer "F.Cu") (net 4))
 (segment (start 144.96 126.04) (end 143.89 124.97) (width 0.75) (layer "F.Cu") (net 4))
 (segment (start 143.89 124.97) (end 137.47 124.97) (width 0.75) (layer "F.Cu") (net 4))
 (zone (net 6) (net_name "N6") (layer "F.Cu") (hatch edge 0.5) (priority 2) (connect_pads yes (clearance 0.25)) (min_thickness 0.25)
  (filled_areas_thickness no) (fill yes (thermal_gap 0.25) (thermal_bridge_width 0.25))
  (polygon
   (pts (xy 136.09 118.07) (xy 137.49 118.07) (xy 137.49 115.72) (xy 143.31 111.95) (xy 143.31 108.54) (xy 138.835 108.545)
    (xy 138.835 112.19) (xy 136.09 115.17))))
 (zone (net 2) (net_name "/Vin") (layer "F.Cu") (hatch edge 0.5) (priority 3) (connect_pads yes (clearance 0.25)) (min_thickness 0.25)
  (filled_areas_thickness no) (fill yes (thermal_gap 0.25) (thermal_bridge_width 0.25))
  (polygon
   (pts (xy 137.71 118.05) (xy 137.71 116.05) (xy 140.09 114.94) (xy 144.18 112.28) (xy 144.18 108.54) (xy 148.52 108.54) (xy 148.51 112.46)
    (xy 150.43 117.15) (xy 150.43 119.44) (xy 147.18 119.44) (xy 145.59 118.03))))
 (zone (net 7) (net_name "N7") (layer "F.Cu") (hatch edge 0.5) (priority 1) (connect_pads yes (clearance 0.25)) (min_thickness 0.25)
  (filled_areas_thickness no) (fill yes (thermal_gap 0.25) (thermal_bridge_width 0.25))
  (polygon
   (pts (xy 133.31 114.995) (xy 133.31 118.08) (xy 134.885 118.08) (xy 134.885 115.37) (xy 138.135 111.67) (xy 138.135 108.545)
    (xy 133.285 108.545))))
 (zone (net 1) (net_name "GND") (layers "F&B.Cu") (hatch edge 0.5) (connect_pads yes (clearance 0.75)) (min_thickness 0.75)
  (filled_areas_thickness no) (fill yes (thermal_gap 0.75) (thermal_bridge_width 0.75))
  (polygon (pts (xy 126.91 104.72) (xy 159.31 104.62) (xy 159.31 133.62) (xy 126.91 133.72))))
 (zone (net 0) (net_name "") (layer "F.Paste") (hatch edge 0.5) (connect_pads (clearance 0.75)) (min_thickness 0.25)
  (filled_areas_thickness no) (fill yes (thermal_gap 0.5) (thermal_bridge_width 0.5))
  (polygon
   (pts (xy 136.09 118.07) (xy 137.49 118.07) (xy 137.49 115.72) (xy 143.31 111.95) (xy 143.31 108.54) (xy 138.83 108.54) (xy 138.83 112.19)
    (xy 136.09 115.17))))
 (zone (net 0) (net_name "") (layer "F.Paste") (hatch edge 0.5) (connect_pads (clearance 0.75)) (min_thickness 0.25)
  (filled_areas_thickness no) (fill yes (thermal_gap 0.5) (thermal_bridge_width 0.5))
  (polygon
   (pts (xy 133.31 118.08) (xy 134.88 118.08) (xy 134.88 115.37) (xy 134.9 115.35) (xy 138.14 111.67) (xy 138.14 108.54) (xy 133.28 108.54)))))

